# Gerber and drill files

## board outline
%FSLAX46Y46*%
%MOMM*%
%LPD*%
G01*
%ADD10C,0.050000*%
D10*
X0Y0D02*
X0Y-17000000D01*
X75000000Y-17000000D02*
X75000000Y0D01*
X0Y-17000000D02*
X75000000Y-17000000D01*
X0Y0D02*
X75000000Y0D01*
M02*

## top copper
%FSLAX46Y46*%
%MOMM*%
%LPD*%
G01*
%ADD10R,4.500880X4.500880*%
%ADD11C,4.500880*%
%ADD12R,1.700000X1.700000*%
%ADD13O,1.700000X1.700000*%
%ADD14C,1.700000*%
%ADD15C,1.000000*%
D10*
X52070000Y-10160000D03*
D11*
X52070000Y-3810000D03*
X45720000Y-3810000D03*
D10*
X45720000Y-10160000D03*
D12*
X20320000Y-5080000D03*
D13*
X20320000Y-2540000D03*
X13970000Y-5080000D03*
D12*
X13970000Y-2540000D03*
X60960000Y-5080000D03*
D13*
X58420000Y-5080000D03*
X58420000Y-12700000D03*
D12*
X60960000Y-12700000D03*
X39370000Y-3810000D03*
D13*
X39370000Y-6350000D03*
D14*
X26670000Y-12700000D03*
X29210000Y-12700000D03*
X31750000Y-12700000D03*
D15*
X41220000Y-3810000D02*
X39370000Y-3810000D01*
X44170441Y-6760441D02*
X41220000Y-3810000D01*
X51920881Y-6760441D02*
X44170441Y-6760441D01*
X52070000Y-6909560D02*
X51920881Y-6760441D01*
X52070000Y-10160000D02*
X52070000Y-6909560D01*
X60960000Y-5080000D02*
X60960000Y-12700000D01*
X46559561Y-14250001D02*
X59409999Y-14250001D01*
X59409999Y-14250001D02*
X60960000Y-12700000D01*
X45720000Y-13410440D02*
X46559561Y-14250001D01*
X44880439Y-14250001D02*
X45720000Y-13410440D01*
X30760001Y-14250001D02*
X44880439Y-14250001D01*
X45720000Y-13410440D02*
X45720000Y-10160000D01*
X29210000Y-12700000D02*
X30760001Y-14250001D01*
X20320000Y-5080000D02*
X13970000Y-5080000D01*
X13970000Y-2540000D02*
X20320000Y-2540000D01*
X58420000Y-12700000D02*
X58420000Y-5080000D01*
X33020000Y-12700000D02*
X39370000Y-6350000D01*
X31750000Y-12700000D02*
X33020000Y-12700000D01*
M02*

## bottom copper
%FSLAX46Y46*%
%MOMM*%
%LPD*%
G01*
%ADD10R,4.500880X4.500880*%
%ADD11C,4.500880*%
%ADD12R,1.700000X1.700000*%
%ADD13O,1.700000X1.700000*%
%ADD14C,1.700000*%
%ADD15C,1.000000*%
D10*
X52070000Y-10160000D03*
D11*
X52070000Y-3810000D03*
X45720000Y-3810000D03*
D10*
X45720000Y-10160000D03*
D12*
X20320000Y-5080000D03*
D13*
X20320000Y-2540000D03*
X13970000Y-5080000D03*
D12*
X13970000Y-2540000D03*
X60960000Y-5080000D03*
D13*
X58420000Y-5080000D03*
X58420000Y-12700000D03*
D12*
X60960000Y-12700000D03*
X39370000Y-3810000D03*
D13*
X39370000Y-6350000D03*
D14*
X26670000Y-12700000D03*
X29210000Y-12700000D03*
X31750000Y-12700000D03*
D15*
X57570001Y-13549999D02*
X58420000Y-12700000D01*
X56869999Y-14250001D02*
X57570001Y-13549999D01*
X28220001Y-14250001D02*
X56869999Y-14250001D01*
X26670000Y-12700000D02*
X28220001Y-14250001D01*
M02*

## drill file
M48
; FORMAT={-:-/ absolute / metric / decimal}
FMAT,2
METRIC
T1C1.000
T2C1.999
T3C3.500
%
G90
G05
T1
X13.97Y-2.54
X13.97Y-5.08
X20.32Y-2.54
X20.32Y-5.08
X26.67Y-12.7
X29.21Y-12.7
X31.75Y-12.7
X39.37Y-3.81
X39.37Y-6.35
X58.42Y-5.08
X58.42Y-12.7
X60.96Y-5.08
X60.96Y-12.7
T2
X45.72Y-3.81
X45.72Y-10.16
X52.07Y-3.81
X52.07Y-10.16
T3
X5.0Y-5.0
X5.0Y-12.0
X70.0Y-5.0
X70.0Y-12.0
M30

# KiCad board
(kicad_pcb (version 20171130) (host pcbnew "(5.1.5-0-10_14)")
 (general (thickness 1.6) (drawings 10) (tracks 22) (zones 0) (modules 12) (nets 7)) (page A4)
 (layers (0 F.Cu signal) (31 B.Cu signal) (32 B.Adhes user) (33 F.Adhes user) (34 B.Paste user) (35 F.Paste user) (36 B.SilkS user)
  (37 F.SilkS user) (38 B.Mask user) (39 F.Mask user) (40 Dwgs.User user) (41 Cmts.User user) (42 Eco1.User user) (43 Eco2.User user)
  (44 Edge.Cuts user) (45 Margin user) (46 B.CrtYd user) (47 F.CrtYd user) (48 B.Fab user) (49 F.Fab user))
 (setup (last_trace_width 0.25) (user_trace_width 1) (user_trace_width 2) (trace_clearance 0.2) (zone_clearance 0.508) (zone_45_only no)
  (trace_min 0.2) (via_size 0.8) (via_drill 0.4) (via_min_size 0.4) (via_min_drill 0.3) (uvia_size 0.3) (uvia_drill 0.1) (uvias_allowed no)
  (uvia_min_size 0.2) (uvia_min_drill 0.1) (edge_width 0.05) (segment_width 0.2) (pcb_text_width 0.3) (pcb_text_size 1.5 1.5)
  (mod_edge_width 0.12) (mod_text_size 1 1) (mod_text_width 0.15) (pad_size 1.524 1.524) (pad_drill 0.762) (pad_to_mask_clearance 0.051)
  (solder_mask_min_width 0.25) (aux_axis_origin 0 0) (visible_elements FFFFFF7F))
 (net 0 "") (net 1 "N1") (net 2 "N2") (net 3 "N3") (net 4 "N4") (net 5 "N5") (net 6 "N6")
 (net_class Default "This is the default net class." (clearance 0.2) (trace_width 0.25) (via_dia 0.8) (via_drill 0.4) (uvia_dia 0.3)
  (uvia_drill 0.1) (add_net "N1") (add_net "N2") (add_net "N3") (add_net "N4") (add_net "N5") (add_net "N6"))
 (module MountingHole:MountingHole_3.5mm (layer F.Cu) (at 70 5)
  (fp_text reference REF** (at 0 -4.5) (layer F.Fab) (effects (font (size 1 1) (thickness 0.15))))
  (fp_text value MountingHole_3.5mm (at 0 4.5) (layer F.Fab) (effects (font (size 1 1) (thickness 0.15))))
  (pad 1 np_thru_hole circle (at 0 0) (size 3.5 3.5) (drill 3.5) (layers *.Cu *.Mask)))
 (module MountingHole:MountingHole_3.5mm (layer F.Cu) (at 70 12)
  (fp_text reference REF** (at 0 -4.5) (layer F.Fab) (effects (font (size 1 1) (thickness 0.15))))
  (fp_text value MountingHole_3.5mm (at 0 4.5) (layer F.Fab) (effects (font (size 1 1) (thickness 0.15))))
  (pad 1 np_thru_hole circle (at 0 0) (size 3.5 3.5) (drill 3.5) (layers *.Cu *.Mask)))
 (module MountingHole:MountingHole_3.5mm (layer F.Cu) (at 5 12)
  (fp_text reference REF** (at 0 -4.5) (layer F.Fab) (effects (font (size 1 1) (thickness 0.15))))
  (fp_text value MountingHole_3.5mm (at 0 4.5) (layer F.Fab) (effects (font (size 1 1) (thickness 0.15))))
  (pad 1 np_thru_hole circle (at 0 0) (size 3.5 3.5) (drill 3.5) (layers *.Cu *.Mask)))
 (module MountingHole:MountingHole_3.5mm (layer F.Cu) (at 5 5)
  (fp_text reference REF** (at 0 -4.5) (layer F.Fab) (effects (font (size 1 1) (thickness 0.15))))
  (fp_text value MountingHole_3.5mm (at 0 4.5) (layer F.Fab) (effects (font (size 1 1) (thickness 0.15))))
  (pad 1 np_thru_hole circle (at 0 0) (size 3.5 3.5) (drill 3.5) (layers *.Cu *.Mask)))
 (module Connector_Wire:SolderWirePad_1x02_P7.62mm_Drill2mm (layer F.Cu) (at 52.07 10.16 90)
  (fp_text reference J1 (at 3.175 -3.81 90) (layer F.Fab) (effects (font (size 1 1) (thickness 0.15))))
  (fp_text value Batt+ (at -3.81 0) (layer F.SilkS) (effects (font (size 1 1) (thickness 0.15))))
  (pad 1 thru_hole rect (at 0 0 90) (size 4.50088 4.50088) (drill 1.99898) (layers *.Cu *.Mask) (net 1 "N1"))
  (pad 2 thru_hole circle (at 6.35 0 90) (size 4.50088 4.50088) (drill 1.99898) (layers *.Cu *.Mask)))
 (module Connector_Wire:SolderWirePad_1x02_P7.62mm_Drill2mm (layer F.Cu) (at 45.72 10.16 90)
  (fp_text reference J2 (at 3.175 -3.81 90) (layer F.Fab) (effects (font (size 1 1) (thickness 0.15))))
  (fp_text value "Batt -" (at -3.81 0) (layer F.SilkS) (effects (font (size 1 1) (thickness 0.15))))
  (pad 2 thru_hole circle (at 6.35 0 90) (size 4.50088 4.50088) (drill 1.99898) (layers *.Cu *.Mask))
  (pad 1 thru_hole rect (at 0 0 90) (size 4.50088 4.50088) (drill 1.99898) (layers *.Cu *.Mask) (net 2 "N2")))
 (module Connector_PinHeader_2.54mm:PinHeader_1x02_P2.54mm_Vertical (layer F.Cu) (at 20.32 5.08 180)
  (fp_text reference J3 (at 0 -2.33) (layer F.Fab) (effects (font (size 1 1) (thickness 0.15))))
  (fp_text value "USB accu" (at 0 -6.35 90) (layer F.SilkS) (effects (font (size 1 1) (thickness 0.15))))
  (pad 1 thru_hole rect (at 0 0 180) (size 1.7 1.7) (drill 1) (layers *.Cu *.Mask) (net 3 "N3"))
  (pad 2 thru_hole oval (at 0 2.54 180) (size 1.7 1.7) (drill 1) (layers *.Cu *.Mask) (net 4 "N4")))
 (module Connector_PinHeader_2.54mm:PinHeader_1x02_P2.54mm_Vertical (layer F.Cu) (at 13.97 2.54)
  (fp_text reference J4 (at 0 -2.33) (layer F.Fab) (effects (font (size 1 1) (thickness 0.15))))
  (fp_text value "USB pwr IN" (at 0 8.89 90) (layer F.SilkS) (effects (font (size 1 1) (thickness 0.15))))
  (pad 2 thru_hole oval (at 0 2.54) (size 1.7 1.7) (drill 1) (layers *.Cu *.Mask) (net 3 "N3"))
  (pad 1 thru_hole rect (at 0 0) (size 1.7 1.7) (drill 1) (layers *.Cu *.Mask) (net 4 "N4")))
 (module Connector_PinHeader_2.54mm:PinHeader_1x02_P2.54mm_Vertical (layer F.Cu) (at 60.96 5.08 270)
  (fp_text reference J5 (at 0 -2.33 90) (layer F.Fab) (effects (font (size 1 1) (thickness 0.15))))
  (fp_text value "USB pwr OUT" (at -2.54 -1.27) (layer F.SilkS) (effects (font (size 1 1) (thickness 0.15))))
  (pad 1 thru_hole rect (at 0 0 270) (size 1.7 1.7) (drill 1) (layers *.Cu *.Mask) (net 2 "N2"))
  (pad 2 thru_hole oval (at 0 2.54 270) (size 1.7 1.7) (drill 1) (layers *.Cu *.Mask) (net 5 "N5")))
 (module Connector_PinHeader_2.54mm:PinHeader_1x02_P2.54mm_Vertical (layer F.Cu) (at 60.96 12.7 270)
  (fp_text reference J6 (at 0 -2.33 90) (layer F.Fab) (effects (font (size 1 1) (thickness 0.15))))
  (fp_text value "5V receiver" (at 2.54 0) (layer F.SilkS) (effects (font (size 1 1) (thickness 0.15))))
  (pad 2 thru_hole oval (at 0 2.54 270) (size 1.7 1.7) (drill 1) (layers *.Cu *.Mask) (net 5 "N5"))
  (pad 1 thru_hole rect (at 0 0 270) (size 1.7 1.7) (drill 1) (layers *.Cu *.Mask) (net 2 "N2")))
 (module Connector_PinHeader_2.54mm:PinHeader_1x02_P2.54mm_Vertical (layer F.Cu) (at 39.37 3.81)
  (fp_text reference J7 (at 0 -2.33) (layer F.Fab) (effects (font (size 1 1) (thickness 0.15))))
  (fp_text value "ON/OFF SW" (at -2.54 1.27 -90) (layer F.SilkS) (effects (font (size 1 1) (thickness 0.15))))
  (pad 1 thru_hole rect (at 0 0) (size 1.7 1.7) (drill 1) (layers *.Cu *.Mask) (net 1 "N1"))
  (pad 2 thru_hole oval (at 0 2.54) (size 1.7 1.7) (drill 1) (layers *.Cu *.Mask) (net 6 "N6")))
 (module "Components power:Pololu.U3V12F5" (layer F.Cu) (at 29.21 7.62)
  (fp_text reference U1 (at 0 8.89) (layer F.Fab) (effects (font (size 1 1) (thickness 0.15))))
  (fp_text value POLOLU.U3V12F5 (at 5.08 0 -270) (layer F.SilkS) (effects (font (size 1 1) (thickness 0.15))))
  (pad 3 thru_hole circle (at -2.54 5.08) (size 1.7 1.7) (drill 1) (layers *.Cu *.Mask) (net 5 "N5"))
  (pad 2 thru_hole circle (at 0 5.08) (size 1.7 1.7) (drill 1) (layers *.Cu *.Mask) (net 2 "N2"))
  (pad 1 thru_hole circle (at 2.54 5.08) (size 1.7 1.7) (drill 1) (layers *.Cu *.Mask) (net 6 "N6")))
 (gr_line (start 0 0) (end 0 17) (layer Edge.Cuts) (width 0.05))
 (gr_line (start 75 17) (end 75 0) (layer Edge.Cuts) (width 0.05))
 (gr_line (start 0 17) (end 75 17) (layer Edge.Cuts) (width 0.05))
 (gr_line (start 0 0) (end 75 0) (layer Edge.Cuts) (width 0.05))
 (segment (start 41.22 3.81) (end 39.37 3.81) (width 1) (layer F.Cu) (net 1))
 (segment (start 44.170441 6.760441) (end 41.22 3.81) (width 1) (layer F.Cu) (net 1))
 (segment (start 51.920881 6.760441) (end 44.170441 6.760441) (width 1) (layer F.Cu) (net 1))
 (segment (start 52.07 6.90956) (end 51.920881 6.760441) (width 1) (layer F.Cu) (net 1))
 (segment (start 52.07 10.16) (end 52.07 6.90956) (width 1) (layer F.Cu) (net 1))
 (segment (start 60.96 5.08) (end 60.96 12.7) (width 1) (layer F.Cu) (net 2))
 (segment (start 46.559561 14.250001) (end 59.409999 14.250001) (width 1) (layer F.Cu) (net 2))
 (segment (start 59.409999 14.250001) (end 60.96 12.7) (width 1) (layer F.Cu) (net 2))
 (segment (start 45.72 13.41044) (end 46.559561 14.250001) (width 1) (layer F.Cu) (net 2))
 (segment (start 44.880439 14.250001) (end 45.72 13.41044) (width 1) (layer F.Cu) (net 2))
 (segment (start 30.760001 14.250001) (end 44.880439 14.250001) (width 1) (layer F.Cu) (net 2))
 (segment (start 45.72 13.41044) (end 45.72 10.16) (width 1) (layer F.Cu) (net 2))
 (segment (start 29.21 12.7) (end 30.760001 14.250001) (width 1) (layer F.Cu) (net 2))
 (segment (start 20.32 5.08) (end 13.97 5.08) (width 1) (layer F.Cu) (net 3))
 (segment (start 13.97 2.54) (end 20.32 2.54) (width 1) (layer F.Cu) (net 4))
 (segment (start 58.42 12.7) (end 58.42 5.08) (width 1) (layer F.Cu) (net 5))
 (segment (start 57.570001 13.549999) (end 58.42 12.7) (width 1) (layer B.Cu) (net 5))
 (segment (start 56.869999 14.250001) (end 57.570001 13.549999) (width 1) (layer B.Cu) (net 5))
 (segment (start 28.220001 14.250001) (end 56.869999 14.250001) (width 1) (layer B.Cu) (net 5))
 (segment (start 26.67 12.7) (end 28.220001 14.250001) (width 1) (layer B.Cu) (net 5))
 (segment (start 33.02 12.7) (end 39.37 6.35) (width 1) (layer F.Cu) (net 6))
 (segment (start 31.75 12.7) (end 33.02 12.7) (width 1) (layer F.Cu) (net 6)))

